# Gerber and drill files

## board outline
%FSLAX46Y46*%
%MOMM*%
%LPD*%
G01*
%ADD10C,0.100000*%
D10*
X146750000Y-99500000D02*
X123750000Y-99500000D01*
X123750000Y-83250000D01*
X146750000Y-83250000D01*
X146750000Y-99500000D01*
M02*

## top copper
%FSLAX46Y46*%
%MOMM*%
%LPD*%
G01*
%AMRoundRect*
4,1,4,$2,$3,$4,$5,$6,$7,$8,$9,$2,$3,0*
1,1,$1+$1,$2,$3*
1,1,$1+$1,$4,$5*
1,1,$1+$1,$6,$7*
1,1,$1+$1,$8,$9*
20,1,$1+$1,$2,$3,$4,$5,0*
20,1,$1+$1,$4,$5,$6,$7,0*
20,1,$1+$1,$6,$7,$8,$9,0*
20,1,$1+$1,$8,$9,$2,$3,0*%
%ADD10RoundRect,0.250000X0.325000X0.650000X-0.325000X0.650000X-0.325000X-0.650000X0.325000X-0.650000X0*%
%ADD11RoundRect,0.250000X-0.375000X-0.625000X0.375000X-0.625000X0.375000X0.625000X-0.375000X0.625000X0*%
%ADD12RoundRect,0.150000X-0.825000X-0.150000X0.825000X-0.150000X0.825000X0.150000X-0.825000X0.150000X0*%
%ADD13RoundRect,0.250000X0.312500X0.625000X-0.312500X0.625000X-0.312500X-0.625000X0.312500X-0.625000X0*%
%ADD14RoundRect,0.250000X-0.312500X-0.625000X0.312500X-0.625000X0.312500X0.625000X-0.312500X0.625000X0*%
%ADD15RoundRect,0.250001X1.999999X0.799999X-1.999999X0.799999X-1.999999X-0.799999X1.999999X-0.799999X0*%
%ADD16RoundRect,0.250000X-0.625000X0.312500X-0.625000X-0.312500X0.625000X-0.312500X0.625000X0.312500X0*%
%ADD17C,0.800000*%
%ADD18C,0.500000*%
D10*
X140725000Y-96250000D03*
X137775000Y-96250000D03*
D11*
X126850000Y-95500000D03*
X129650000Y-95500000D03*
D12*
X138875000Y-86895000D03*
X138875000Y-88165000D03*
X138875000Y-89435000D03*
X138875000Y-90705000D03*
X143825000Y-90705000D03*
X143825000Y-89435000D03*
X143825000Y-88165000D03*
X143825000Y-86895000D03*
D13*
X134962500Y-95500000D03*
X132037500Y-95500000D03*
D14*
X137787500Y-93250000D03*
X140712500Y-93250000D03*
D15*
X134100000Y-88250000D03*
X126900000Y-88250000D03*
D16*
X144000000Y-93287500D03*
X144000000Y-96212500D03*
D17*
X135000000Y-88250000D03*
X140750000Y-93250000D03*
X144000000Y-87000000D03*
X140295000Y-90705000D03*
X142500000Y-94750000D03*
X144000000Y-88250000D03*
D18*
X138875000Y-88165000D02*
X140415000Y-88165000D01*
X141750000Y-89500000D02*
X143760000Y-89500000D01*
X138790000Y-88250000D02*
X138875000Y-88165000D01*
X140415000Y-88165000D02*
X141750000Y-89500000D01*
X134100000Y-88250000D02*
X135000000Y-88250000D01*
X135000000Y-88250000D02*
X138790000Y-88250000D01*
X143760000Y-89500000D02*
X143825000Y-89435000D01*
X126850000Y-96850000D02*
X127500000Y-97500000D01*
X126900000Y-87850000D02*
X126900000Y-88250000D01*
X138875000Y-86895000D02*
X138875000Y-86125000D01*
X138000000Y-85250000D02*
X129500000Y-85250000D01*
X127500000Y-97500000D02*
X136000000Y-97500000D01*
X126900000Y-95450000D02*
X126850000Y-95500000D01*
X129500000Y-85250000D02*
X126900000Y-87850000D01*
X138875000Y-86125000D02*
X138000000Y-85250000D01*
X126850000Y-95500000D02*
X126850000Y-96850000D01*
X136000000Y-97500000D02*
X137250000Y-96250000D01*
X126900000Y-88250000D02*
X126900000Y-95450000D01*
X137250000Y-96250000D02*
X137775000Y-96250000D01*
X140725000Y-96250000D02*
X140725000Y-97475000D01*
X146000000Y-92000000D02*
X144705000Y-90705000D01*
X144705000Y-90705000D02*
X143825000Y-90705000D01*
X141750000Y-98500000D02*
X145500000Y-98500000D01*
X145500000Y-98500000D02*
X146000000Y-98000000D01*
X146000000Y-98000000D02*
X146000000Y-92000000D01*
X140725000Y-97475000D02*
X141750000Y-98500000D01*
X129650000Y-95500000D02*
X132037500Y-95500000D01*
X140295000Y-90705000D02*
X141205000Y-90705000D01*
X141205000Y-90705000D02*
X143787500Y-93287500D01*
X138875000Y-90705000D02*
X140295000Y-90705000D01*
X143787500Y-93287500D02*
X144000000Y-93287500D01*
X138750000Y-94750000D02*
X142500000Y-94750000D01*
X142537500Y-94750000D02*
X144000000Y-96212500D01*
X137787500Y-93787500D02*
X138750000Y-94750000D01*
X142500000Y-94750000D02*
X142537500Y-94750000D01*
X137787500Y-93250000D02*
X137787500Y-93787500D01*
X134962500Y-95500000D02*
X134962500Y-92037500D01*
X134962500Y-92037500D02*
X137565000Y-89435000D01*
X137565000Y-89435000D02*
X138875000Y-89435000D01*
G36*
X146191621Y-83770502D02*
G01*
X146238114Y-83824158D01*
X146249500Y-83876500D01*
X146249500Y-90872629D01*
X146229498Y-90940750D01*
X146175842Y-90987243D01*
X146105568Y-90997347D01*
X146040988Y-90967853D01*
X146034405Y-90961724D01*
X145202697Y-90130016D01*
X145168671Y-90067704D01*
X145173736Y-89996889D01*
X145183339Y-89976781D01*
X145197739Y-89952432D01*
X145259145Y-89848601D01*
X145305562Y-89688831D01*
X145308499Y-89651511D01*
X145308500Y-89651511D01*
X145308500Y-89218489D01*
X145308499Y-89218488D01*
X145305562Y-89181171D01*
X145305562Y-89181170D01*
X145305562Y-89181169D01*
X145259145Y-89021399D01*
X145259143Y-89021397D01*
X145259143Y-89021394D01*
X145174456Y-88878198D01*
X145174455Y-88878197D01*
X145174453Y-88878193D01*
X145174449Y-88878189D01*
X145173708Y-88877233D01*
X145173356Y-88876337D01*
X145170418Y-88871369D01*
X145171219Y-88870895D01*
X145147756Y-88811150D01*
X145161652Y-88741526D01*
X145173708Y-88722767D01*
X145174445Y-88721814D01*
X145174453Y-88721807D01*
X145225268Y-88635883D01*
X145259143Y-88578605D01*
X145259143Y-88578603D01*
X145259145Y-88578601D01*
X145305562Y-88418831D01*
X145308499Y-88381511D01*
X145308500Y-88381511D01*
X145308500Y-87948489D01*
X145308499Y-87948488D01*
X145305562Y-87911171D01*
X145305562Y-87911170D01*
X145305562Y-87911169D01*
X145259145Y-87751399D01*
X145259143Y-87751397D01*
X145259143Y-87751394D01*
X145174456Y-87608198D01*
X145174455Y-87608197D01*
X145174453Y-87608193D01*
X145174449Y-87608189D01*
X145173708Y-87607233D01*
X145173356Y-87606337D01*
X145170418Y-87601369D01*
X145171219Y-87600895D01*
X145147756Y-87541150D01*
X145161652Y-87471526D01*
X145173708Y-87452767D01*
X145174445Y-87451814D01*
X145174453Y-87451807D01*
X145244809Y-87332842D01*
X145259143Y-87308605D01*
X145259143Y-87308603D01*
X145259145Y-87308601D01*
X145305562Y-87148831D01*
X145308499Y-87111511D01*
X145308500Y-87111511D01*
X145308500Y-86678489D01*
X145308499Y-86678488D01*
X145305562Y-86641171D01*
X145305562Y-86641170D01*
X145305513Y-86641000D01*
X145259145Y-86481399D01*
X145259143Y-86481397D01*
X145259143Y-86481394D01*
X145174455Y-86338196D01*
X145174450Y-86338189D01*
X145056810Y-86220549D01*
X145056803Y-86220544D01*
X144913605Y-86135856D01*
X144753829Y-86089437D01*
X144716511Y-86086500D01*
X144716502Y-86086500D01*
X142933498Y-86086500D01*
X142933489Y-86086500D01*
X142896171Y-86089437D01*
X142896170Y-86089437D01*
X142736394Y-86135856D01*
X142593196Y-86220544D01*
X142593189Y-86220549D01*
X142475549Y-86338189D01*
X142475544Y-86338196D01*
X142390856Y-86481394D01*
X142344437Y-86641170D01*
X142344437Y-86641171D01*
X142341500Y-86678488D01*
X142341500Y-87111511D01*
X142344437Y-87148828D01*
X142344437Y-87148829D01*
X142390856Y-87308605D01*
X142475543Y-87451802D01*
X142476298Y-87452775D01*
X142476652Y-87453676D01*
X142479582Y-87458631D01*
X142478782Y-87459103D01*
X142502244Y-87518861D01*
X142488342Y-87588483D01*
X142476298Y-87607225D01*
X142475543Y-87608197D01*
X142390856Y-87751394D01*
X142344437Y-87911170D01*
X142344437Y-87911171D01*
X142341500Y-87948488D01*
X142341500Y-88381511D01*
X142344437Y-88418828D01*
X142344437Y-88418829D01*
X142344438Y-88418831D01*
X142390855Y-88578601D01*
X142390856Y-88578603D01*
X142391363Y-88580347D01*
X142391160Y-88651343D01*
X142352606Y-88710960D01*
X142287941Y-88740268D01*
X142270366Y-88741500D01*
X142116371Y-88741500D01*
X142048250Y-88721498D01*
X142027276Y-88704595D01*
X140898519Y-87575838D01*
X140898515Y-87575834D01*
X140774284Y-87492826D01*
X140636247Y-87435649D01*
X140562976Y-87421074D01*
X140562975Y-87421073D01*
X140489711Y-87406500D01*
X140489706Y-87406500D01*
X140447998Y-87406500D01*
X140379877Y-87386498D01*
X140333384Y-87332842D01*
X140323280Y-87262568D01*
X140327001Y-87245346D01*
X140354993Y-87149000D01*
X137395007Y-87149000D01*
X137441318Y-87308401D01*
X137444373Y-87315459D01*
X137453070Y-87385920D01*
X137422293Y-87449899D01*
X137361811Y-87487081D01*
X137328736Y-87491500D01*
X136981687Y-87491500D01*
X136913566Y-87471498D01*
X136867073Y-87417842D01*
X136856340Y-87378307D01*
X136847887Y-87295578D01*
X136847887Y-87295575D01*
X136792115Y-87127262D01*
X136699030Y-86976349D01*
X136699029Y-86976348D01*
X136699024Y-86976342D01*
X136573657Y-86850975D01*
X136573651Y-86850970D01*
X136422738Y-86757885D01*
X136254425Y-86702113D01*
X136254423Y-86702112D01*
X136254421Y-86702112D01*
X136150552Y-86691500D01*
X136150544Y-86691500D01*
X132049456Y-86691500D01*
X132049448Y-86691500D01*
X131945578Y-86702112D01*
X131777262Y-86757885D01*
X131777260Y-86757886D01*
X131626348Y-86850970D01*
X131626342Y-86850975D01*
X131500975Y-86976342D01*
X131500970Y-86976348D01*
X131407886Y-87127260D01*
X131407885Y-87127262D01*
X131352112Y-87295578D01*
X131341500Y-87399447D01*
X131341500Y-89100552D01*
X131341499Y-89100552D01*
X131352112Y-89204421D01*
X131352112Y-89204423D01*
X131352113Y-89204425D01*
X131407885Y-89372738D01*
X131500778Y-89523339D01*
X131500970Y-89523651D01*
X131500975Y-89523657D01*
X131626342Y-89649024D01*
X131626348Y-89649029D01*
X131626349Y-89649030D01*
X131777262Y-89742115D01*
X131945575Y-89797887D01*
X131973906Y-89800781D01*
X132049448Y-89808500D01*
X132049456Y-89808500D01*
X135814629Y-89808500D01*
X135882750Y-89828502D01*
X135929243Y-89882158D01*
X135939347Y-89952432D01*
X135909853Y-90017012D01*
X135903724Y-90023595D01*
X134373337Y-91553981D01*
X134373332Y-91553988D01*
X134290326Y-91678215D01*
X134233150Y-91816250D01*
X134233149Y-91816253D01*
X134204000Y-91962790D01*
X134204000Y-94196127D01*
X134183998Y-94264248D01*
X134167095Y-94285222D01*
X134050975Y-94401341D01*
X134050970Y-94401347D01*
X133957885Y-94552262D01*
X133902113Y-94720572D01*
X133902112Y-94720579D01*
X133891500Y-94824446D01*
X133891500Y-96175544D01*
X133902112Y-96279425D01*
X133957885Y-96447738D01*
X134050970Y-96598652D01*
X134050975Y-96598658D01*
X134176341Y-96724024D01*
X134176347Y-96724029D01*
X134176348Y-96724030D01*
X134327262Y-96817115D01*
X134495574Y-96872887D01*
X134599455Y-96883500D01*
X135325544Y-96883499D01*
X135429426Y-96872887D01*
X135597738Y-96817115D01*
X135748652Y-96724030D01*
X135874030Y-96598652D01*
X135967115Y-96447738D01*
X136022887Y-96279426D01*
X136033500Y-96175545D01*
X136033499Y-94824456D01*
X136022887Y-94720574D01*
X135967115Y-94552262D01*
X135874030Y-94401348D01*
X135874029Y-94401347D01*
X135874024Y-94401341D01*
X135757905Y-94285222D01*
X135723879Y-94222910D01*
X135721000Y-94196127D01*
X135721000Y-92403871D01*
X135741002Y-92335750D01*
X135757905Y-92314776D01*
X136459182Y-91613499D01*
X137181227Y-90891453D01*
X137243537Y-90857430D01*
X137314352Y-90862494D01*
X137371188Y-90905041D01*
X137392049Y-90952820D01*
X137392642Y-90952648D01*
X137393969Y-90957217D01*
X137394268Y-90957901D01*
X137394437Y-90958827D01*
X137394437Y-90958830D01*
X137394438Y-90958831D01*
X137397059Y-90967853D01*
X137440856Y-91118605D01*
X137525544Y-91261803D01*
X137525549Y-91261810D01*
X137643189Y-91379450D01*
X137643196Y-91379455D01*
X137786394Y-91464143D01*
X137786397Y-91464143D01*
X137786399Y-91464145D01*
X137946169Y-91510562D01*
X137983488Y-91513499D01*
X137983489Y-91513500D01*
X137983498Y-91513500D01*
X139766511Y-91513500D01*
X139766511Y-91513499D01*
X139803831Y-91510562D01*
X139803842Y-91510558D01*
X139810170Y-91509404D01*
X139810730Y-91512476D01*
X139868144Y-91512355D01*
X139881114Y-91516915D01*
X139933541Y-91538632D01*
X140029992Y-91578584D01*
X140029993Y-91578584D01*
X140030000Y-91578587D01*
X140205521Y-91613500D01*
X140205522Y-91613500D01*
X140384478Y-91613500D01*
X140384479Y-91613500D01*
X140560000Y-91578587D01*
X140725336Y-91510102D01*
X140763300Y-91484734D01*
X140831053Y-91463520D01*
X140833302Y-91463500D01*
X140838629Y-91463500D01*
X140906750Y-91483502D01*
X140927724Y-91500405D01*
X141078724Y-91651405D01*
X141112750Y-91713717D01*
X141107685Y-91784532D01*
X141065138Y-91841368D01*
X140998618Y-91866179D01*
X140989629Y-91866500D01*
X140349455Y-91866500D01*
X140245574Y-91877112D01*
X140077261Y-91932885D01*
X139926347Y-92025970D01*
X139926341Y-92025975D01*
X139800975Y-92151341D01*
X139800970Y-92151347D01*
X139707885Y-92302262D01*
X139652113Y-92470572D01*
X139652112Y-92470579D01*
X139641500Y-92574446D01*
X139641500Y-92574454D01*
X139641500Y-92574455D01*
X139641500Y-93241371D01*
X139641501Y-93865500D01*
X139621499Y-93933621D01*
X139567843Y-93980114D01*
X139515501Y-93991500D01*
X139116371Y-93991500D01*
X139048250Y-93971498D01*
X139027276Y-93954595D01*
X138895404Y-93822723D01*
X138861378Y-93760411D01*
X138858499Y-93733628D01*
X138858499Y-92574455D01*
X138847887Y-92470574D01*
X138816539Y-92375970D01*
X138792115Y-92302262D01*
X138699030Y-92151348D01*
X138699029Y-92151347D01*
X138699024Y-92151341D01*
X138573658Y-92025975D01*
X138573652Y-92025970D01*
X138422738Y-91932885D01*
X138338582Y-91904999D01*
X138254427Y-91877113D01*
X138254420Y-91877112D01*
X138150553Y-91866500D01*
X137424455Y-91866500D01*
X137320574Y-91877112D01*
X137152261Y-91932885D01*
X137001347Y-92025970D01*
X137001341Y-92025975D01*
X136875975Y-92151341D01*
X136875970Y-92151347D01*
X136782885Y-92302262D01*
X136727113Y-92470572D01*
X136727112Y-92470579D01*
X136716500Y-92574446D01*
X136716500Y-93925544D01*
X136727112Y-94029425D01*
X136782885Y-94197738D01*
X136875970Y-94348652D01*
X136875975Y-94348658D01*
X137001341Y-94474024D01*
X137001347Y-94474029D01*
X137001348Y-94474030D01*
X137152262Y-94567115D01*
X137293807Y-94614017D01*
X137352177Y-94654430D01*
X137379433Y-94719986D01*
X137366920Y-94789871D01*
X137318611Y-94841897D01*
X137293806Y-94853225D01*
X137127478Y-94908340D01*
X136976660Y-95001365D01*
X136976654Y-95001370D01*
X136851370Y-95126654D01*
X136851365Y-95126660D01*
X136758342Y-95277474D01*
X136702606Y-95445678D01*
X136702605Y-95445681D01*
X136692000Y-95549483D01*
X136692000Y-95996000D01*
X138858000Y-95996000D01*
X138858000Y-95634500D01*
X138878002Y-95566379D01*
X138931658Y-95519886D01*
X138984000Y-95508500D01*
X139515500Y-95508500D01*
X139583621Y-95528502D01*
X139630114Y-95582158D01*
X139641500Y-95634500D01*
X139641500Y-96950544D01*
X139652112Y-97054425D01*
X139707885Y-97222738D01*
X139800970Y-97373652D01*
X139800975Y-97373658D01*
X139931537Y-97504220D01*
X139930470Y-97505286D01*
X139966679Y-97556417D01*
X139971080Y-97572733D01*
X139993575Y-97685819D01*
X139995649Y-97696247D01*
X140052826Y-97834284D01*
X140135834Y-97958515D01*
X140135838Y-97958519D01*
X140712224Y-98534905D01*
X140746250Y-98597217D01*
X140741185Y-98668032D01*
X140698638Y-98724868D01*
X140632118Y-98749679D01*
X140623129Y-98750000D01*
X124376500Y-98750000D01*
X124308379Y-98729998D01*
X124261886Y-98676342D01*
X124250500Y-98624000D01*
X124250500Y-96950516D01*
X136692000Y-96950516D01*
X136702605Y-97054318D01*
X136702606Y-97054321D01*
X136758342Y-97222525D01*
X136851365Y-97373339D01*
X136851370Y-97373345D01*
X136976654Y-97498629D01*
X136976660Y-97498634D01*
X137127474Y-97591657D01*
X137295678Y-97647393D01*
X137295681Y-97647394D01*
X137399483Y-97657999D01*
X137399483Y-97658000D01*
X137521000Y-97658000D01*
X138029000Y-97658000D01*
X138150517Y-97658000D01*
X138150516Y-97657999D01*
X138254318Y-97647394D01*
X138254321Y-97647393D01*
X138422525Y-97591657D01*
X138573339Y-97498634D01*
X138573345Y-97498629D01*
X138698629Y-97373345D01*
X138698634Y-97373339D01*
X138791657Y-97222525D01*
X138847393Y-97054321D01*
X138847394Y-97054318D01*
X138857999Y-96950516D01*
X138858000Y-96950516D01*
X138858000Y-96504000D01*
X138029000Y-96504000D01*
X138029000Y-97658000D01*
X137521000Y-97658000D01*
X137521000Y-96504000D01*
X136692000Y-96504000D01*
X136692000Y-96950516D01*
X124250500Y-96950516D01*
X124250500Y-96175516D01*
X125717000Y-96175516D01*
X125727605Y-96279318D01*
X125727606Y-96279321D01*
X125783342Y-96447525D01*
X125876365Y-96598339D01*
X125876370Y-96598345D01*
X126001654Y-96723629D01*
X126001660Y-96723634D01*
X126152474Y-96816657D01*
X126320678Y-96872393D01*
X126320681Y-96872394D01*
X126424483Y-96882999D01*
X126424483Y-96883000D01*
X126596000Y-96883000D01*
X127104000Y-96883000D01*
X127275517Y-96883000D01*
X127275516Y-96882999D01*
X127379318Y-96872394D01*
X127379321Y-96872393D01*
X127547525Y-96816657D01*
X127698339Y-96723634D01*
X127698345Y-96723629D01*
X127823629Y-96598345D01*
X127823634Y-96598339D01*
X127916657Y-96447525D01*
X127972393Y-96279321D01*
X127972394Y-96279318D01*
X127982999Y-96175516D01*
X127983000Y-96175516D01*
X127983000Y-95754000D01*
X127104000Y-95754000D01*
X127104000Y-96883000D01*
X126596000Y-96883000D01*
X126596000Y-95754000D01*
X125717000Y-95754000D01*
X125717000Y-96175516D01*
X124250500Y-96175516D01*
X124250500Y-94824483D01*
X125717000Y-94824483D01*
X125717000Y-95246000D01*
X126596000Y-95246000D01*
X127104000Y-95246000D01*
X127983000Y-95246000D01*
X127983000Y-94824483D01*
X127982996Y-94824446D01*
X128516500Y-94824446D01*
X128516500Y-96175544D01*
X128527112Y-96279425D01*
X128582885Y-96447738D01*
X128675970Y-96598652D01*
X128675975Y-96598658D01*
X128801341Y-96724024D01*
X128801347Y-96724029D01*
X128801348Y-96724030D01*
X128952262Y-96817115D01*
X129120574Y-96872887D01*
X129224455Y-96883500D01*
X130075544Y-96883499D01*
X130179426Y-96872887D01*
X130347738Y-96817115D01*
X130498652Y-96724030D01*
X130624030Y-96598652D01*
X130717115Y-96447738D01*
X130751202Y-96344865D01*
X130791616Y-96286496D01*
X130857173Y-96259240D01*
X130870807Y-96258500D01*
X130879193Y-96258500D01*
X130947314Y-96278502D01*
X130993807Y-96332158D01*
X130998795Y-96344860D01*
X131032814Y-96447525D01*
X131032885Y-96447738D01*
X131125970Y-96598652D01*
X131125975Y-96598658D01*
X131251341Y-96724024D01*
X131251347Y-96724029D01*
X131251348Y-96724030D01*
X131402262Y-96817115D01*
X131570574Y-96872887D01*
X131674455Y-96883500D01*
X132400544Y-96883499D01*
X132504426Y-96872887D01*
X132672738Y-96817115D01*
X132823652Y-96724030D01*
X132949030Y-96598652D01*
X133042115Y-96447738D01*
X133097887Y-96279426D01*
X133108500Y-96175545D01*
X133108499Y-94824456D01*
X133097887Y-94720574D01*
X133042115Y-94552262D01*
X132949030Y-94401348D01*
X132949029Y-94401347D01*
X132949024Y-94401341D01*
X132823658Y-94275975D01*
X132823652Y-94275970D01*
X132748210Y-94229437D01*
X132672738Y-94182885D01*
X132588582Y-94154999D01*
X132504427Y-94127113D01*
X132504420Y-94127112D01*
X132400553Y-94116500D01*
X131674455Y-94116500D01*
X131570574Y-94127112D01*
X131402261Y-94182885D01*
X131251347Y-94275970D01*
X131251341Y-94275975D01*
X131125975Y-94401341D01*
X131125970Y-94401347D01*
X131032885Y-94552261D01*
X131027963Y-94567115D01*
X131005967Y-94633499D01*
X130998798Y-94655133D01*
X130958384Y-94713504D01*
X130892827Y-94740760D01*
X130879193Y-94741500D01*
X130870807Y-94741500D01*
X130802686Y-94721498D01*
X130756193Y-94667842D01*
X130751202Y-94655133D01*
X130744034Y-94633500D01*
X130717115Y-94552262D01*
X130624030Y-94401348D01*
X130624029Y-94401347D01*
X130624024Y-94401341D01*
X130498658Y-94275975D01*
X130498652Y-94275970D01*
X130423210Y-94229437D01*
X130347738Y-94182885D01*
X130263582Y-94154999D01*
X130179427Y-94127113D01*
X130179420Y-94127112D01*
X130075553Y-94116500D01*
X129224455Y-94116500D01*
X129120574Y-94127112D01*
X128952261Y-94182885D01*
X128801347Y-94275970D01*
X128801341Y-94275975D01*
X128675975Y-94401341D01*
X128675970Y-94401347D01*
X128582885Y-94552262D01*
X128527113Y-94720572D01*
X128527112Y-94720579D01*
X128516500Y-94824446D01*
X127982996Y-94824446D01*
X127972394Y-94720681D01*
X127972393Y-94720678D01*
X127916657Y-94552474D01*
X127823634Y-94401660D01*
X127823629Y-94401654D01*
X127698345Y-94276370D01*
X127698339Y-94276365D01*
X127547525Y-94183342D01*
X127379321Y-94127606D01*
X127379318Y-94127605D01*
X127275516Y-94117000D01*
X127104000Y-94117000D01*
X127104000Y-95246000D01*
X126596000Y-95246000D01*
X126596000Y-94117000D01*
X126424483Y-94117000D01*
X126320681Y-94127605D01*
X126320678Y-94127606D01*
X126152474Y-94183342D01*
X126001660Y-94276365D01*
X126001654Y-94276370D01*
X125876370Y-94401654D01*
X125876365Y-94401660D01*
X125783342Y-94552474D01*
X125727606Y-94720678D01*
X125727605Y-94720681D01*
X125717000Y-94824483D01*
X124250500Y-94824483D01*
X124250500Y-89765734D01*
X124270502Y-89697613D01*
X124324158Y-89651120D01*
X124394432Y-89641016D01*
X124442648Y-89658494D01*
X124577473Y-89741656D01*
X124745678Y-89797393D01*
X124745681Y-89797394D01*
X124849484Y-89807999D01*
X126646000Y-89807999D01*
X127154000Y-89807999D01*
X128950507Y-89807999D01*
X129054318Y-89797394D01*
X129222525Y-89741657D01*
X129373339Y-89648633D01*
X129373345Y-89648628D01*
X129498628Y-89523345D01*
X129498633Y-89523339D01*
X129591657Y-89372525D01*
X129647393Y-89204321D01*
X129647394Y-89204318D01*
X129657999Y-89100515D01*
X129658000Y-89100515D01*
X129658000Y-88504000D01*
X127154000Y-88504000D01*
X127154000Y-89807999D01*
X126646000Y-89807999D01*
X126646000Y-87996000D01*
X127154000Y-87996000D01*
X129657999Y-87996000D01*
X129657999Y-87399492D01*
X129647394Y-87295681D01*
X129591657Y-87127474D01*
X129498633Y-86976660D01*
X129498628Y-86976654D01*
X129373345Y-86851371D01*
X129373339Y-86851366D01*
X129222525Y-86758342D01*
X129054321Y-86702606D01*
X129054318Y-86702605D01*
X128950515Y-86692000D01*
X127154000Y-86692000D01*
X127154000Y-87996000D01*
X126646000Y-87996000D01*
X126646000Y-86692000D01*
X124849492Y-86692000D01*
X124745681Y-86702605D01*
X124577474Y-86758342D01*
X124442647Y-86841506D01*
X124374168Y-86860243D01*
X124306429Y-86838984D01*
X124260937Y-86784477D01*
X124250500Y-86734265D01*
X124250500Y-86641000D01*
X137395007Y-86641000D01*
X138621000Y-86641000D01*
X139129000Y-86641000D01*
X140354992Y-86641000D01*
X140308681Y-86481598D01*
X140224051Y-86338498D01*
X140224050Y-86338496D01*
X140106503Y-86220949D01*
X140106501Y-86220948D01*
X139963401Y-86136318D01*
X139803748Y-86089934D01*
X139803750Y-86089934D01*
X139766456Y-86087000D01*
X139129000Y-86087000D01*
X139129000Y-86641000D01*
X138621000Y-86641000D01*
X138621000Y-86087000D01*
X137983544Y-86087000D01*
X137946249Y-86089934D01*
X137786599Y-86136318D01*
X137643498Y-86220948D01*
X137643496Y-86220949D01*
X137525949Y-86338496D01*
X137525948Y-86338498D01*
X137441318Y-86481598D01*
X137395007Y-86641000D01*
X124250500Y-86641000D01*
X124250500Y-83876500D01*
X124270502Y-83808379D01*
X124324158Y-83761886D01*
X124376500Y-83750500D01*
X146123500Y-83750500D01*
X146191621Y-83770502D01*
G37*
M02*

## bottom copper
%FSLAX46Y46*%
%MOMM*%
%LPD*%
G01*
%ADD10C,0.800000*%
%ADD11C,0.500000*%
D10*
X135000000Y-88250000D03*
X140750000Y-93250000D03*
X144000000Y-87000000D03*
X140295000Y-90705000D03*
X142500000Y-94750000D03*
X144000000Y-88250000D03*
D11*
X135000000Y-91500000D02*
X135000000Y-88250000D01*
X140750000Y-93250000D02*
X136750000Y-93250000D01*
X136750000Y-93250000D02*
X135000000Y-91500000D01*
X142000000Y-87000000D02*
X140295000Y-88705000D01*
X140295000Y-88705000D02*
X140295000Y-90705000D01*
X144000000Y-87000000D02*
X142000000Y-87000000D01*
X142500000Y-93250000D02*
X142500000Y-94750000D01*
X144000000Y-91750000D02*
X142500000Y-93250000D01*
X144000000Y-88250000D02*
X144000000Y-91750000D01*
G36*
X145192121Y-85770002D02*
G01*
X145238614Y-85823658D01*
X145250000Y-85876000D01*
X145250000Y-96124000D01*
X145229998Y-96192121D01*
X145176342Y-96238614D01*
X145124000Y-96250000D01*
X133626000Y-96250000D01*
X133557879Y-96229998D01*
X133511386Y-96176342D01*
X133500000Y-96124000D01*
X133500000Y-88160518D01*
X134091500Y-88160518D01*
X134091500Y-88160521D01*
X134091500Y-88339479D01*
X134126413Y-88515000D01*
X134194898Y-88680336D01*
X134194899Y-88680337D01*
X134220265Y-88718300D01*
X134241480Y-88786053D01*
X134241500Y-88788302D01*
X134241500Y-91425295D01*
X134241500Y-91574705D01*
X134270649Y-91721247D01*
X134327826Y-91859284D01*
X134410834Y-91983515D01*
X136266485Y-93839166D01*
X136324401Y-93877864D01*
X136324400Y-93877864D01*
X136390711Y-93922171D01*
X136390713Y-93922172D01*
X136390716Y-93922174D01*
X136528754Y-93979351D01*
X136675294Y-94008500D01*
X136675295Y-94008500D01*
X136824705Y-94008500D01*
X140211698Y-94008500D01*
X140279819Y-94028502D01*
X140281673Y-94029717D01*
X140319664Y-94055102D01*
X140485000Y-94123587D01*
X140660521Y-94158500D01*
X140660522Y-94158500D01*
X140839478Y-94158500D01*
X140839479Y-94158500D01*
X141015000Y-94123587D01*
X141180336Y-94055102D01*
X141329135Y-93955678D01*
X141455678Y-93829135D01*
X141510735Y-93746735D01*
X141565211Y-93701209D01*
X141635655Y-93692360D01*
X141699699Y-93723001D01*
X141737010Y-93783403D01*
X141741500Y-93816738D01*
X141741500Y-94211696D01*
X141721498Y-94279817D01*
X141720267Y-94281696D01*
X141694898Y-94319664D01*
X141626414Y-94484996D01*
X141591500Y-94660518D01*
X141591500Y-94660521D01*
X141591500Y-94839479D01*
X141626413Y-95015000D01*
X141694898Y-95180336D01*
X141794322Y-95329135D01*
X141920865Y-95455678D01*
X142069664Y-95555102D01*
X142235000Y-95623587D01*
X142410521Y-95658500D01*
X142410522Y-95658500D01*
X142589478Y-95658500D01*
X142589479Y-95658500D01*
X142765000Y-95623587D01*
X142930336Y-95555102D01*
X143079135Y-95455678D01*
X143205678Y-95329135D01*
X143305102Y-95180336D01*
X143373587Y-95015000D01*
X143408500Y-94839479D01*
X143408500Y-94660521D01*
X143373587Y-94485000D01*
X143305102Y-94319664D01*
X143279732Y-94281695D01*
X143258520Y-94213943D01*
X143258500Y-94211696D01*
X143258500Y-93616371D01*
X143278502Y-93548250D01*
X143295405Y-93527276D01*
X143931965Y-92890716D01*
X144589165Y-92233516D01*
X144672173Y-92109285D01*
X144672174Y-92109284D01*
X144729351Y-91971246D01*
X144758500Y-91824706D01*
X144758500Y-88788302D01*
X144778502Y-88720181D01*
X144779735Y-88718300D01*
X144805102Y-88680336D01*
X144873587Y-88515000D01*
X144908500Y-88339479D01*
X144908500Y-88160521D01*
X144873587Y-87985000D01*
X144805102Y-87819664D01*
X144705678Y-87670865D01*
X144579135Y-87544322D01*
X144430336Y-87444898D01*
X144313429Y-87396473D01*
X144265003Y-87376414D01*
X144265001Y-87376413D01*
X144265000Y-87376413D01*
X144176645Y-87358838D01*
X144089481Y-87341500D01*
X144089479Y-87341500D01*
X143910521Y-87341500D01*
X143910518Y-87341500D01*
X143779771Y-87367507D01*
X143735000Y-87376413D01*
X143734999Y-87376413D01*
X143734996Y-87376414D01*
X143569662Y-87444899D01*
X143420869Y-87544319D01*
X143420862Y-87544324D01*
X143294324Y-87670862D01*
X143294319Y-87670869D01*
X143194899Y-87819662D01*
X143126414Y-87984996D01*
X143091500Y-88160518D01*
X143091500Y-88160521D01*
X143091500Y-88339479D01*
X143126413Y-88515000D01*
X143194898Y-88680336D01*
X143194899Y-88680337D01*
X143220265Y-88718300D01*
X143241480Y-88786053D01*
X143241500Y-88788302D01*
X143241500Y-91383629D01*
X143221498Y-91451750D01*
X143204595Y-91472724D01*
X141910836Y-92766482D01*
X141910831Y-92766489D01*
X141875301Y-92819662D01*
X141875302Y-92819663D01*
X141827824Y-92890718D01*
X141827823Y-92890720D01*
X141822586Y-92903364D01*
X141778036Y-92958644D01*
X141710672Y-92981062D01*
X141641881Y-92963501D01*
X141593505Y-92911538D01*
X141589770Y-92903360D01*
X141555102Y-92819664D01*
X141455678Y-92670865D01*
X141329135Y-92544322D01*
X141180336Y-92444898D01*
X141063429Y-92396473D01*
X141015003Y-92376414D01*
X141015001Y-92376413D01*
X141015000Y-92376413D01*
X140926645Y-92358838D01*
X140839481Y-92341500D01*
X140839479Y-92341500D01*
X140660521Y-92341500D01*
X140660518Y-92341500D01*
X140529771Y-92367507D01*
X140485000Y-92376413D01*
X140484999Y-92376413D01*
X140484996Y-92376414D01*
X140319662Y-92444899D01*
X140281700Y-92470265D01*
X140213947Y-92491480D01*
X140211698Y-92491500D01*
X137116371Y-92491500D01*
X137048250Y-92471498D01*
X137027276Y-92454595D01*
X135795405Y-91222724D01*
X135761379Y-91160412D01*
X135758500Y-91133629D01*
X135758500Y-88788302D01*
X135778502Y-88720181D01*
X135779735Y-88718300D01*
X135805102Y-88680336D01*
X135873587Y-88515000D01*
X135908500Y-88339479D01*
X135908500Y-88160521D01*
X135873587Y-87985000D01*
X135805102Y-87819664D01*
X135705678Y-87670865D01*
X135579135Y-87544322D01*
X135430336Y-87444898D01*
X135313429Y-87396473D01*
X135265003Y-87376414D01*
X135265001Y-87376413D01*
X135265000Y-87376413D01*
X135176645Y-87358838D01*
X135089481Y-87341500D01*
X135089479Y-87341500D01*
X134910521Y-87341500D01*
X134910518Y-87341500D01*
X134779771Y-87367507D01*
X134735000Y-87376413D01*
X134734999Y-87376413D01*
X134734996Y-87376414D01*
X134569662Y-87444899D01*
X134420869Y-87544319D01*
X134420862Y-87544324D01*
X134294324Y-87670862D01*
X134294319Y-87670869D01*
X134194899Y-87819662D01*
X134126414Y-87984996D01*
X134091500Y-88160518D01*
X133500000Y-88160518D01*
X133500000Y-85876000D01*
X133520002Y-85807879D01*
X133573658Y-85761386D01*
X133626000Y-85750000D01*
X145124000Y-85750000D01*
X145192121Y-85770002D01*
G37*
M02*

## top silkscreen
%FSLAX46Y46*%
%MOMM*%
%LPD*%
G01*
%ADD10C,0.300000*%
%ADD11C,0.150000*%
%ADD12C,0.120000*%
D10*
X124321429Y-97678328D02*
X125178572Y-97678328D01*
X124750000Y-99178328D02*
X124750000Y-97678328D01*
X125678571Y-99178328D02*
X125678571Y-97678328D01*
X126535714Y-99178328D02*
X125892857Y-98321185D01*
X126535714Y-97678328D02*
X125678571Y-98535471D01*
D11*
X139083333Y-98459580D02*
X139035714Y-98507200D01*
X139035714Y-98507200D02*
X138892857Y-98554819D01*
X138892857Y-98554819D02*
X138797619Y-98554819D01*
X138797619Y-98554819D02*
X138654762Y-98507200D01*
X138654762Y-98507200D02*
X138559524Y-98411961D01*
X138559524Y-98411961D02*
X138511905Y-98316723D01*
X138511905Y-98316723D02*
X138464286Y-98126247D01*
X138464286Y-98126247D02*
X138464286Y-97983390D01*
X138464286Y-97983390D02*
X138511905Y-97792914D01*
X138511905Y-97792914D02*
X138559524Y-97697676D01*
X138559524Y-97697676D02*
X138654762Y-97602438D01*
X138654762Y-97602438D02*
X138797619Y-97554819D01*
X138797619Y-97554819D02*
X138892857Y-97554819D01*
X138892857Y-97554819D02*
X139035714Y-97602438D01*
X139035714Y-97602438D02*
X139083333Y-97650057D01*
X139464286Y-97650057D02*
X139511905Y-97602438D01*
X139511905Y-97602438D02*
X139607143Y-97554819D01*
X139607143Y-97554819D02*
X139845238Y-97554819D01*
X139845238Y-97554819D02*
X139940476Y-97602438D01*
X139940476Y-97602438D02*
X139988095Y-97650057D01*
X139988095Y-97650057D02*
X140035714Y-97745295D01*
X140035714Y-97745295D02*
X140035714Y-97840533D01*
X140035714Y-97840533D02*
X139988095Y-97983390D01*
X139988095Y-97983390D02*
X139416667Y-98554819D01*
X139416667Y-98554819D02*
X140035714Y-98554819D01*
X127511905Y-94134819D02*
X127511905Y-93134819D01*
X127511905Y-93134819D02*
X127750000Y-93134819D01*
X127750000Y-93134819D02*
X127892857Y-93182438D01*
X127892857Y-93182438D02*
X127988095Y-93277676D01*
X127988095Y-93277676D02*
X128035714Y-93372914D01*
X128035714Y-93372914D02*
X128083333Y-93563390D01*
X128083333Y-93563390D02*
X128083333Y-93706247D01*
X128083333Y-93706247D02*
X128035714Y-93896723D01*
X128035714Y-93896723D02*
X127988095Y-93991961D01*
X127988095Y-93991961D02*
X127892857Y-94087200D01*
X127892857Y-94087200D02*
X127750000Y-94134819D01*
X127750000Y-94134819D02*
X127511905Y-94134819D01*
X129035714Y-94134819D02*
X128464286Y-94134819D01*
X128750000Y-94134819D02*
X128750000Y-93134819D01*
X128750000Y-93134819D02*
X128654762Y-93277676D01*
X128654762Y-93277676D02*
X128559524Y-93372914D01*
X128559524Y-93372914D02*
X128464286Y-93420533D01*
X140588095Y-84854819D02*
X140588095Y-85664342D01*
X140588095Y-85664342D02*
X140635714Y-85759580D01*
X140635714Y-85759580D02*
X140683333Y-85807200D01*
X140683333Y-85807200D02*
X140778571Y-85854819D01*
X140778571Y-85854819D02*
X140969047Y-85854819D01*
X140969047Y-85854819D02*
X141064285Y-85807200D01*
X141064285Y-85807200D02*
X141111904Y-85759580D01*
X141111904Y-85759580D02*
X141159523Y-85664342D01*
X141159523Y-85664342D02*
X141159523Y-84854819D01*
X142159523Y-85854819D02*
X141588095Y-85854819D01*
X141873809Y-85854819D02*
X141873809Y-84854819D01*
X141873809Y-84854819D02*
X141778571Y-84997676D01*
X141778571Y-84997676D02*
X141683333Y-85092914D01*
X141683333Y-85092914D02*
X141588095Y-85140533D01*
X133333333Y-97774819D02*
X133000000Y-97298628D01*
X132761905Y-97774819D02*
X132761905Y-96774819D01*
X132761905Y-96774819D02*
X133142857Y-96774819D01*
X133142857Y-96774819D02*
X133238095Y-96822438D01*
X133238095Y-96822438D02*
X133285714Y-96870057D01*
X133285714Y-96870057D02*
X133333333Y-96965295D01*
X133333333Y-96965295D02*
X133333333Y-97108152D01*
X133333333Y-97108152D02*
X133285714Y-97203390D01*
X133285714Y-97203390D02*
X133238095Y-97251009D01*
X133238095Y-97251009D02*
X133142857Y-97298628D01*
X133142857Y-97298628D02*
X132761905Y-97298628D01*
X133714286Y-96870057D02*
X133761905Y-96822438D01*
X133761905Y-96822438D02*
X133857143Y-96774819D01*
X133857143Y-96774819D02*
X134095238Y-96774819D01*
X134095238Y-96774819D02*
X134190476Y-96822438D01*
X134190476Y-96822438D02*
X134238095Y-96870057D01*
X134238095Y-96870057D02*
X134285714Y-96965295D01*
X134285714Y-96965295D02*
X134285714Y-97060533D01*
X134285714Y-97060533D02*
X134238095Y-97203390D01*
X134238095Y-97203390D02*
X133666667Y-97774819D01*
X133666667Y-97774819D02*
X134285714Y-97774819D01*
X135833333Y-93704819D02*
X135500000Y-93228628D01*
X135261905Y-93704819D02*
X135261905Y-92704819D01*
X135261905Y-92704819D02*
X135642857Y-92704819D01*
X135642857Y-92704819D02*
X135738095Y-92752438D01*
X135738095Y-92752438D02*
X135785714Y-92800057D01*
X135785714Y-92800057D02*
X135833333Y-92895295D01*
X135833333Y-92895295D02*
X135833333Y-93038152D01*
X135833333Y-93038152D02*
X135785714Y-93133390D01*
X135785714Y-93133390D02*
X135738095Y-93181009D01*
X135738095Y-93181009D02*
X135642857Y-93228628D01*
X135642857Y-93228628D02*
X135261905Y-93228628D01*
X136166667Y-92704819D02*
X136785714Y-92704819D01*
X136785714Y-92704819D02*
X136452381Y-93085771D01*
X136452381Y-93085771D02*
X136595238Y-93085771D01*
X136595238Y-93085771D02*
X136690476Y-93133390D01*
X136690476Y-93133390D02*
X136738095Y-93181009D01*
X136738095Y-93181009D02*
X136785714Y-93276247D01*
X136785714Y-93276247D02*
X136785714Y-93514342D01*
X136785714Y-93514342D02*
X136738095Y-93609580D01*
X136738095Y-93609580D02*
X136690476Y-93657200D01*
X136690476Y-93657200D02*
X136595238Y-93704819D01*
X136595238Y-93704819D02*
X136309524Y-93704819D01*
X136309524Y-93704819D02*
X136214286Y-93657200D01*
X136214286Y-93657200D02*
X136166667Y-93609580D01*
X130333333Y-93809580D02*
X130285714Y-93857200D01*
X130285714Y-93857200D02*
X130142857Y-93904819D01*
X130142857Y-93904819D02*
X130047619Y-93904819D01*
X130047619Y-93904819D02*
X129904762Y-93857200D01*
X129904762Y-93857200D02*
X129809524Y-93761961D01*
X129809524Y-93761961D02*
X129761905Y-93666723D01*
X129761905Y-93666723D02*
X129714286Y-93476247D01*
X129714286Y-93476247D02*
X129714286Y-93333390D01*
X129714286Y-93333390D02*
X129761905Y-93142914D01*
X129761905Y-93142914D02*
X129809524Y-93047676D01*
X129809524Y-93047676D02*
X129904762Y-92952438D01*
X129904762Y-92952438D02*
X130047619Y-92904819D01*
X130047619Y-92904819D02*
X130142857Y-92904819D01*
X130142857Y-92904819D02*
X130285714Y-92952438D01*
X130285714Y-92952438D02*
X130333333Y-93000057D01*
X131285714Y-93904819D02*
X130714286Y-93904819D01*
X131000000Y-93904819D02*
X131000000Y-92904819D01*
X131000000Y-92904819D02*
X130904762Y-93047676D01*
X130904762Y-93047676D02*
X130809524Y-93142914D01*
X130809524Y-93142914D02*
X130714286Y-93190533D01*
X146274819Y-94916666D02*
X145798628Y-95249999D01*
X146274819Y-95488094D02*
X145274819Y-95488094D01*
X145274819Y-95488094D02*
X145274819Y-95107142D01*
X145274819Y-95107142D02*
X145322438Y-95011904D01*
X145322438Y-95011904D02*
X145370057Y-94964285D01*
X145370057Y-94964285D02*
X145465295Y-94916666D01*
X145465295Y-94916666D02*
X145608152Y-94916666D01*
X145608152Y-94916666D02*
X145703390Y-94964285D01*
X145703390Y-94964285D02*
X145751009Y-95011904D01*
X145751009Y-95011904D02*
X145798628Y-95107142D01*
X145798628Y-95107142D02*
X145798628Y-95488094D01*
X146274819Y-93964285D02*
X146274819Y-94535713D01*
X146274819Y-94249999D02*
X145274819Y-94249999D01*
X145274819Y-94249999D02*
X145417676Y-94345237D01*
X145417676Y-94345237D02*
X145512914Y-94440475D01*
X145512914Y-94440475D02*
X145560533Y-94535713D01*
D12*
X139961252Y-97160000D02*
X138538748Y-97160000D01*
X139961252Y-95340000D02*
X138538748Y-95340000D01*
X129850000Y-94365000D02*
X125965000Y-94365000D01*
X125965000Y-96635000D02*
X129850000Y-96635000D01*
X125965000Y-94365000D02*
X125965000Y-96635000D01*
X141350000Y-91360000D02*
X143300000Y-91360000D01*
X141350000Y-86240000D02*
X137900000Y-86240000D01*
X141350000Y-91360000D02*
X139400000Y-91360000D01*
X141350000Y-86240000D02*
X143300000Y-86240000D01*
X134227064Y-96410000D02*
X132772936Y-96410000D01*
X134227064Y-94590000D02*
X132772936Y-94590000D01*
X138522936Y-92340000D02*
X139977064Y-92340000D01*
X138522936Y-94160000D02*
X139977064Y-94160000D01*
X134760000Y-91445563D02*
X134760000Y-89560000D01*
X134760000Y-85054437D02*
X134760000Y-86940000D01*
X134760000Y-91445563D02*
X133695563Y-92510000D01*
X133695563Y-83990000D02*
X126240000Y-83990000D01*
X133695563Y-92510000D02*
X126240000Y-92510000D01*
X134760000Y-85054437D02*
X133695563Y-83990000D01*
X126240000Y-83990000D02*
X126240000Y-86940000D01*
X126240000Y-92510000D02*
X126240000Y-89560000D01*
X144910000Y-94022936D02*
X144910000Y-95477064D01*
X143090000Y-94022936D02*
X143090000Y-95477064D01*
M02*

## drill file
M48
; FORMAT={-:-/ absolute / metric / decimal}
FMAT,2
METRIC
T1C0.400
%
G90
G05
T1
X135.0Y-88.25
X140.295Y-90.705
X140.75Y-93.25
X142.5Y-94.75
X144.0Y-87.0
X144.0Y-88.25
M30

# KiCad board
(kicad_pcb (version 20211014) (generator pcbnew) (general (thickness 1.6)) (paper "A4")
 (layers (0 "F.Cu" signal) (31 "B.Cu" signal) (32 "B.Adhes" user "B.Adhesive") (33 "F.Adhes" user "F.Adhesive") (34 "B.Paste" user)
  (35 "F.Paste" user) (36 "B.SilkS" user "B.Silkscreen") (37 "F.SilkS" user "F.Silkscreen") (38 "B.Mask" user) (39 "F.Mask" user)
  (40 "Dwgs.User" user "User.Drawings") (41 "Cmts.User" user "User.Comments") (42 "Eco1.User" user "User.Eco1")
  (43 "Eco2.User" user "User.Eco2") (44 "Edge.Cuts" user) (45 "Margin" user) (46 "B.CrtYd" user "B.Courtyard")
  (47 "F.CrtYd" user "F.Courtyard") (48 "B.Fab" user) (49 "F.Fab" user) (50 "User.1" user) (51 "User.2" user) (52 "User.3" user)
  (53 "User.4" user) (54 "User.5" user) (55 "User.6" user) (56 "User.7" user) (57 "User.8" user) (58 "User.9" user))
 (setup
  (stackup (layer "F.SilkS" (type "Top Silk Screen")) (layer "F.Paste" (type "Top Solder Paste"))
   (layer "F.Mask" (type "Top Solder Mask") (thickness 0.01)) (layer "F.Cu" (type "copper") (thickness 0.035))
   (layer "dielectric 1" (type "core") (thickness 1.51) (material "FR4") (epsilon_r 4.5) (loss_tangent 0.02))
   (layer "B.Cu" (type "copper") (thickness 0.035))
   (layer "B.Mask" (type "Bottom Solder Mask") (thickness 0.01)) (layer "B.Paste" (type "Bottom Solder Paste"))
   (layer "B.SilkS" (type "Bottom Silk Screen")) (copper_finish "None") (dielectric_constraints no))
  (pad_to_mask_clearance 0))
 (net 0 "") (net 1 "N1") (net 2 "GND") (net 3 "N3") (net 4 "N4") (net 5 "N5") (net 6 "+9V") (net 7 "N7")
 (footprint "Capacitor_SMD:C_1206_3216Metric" (layer "F.Cu") (at 139.25 96.25 180)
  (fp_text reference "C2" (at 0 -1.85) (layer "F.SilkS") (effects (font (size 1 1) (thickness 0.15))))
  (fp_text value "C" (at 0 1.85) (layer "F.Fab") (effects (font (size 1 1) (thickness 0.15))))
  (fp_line (start -0.711252 -0.91) (end 0.711252 -0.91) (layer "F.SilkS") (width 0.12))
  (fp_line (start -0.711252 0.91) (end 0.711252 0.91) (layer "F.SilkS") (width 0.12))
  (pad "1" smd roundrect (at -1.475 0 180) (size 1.15 1.8) (layers "F.Cu" "F.Paste" "F.Mask") (roundrect_rratio 0.2173913043) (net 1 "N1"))
  (pad "2" smd roundrect (at 1.475 0 180) (size 1.15 1.8) (layers "F.Cu" "F.Paste" "F.Mask") (roundrect_rratio 0.2173913043) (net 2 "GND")))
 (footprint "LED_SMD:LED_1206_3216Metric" (layer "F.Cu") (at 128.25 95.5)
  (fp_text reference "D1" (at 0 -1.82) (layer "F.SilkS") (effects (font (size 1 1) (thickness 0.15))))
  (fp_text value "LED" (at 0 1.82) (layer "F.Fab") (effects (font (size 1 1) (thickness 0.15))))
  (fp_line (start 1.6 -1.135) (end -2.285 -1.135) (layer "F.SilkS") (width 0.12))
  (fp_line (start -2.285 1.135) (end 1.6 1.135) (layer "F.SilkS") (width 0.12))
  (fp_line (start -2.285 -1.135) (end -2.285 1.135) (layer "F.SilkS") (width 0.12))
  (pad "1" smd roundrect (at -1.4 0) (size 1.25 1.75) (layers "F.Cu" "F.Paste" "F.Mask") (roundrect_rratio 0.2) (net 2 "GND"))
  (pad "2" smd roundrect (at 1.4 0) (size 1.25 1.75) (layers "F.Cu" "F.Paste" "F.Mask") (roundrect_rratio 0.2) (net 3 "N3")))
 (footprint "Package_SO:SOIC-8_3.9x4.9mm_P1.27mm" (layer "F.Cu") (at 141.35 88.8)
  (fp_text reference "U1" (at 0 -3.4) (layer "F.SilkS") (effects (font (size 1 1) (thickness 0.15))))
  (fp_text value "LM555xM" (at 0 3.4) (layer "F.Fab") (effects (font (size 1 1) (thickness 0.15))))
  (fp_line (start 0 2.56) (end 1.95 2.56) (layer "F.SilkS") (width 0.12))
  (fp_line (start 0 -2.56) (end -3.45 -2.56) (layer "F.SilkS") (width 0.12))
  (fp_line (start 0 2.56) (end -1.95 2.56) (layer "F.SilkS") (width 0.12))
  (fp_line (start 0 -2.56) (end 1.95 -2.56) (layer "F.SilkS") (width 0.12))
  (pad "1" smd roundrect (at -2.475 -1.905) (size 1.95 0.6) (layers "F.Cu" "F.Paste" "F.Mask") (roundrect_rratio 0.25) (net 2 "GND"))
  (pad "2" smd roundrect (at -2.475 -0.635) (size 1.95 0.6) (layers "F.Cu" "F.Paste" "F.Mask") (roundrect_rratio 0.25) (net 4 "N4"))
  (pad "3" smd roundrect (at -2.475 0.635) (size 1.95 0.6) (layers "F.Cu" "F.Paste" "F.Mask") (roundrect_rratio 0.25) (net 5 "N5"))
  (pad "4" smd roundrect (at -2.475 1.905) (size 1.95 0.6) (layers "F.Cu" "F.Paste" "F.Mask") (roundrect_rratio 0.25) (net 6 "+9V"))
  (pad "5" smd roundrect (at 2.475 1.905) (size 1.95 0.6) (layers "F.Cu" "F.Paste" "F.Mask") (roundrect_rratio 0.25) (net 1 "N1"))
  (pad "6" smd roundrect (at 2.475 0.635) (size 1.95 0.6) (layers "F.Cu" "F.Paste" "F.Mask") (roundrect_rratio 0.25) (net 4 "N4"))
  (pad "7" smd roundrect (at 2.475 -0.635) (size 1.95 0.6) (layers "F.Cu" "F.Paste" "F.Mask") (roundrect_rratio 0.25) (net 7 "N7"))
  (pad "8" smd roundrect (at 2.475 -1.905) (size 1.95 0.6) (layers "F.Cu" "F.Paste" "F.Mask") (roundrect_rratio 0.25) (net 6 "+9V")))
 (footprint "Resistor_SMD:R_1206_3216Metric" (layer "F.Cu") (at 133.5 95.5 180)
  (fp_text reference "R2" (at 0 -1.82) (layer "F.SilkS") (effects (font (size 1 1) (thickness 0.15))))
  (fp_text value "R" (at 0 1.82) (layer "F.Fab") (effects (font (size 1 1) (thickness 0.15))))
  (fp_line (start -0.727064 -0.91) (end 0.727064 -0.91) (layer "F.SilkS") (width 0.12))
  (fp_line (start -0.727064 0.91) (end 0.727064 0.91) (layer "F.SilkS") (width 0.12))
  (pad "1" smd roundrect (at -1.4625 0 180) (size 1.125 1.75) (layers "F.Cu" "F.Paste" "F.Mask") (roundrect_rratio 0.2222222222)
   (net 5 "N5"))
  (pad "2" smd roundrect (at 1.4625 0 180) (size 1.125 1.75) (layers "F.Cu" "F.Paste" "F.Mask") (roundrect_rratio 0.2222222222) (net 3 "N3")))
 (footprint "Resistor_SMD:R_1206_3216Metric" (layer "F.Cu") (at 139.25 93.25)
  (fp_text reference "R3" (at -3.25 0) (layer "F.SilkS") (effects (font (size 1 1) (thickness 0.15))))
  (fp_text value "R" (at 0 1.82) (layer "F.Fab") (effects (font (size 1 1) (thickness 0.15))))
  (fp_line (start -0.727064 -0.91) (end 0.727064 -0.91) (layer "F.SilkS") (width 0.12))
  (fp_line (start -0.727064 0.91) (end 0.727064 0.91) (layer "F.SilkS") (width 0.12))
  (pad "1" smd roundrect (at -1.4625 0) (size 1.125 1.75) (layers "F.Cu" "F.Paste" "F.Mask") (roundrect_rratio 0.2222222222) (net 7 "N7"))
  (pad "2" smd roundrect (at 1.4625 0) (size 1.125 1.75) (layers "F.Cu" "F.Paste" "F.Mask") (roundrect_rratio 0.2222222222) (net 4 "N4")))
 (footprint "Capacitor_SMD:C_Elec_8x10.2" (layer "F.Cu") (at 130.5 88.25 180)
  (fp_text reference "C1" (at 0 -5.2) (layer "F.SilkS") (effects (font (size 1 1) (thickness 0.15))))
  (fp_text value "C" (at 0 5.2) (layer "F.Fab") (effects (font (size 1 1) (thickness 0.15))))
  (fp_line (start -4.26 -3.195563) (end -4.26 -1.31) (layer "F.SilkS") (width 0.12))
  (fp_line (start -4.26 3.195563) (end -4.26 1.31) (layer "F.SilkS") (width 0.12))
  (fp_line (start -4.26 -3.195563) (end -3.195563 -4.26) (layer "F.SilkS") (width 0.12))
  (fp_line (start -3.195563 4.26) (end 4.26 4.26) (layer "F.SilkS") (width 0.12))
  (fp_line (start -3.195563 -4.26) (end 4.26 -4.26) (layer "F.SilkS") (width 0.12))
  (fp_line (start -4.26 3.195563) (end -3.195563 4.26) (layer "F.SilkS") (width 0.12))
  (fp_line (start 4.26 4.26) (end 4.26 1.31) (layer "F.SilkS") (width 0.12))
  (fp_line (start 4.26 -4.26) (end 4.26 -1.31) (layer "F.SilkS") (width 0.12))
  (pad "1" smd roundrect (at -3.6 0 180) (size 4.5 2.1) (layers "F.Cu" "F.Paste" "F.Mask") (roundrect_rratio 0.1190480952) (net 4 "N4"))
  (pad "2" smd roundrect (at 3.6 0 180) (size 4.5 2.1) (layers "F.Cu" "F.Paste" "F.Mask") (roundrect_rratio 0.1190480952) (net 2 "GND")))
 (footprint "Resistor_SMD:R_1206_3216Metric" (layer "F.Cu") (at 144 94.75 -90)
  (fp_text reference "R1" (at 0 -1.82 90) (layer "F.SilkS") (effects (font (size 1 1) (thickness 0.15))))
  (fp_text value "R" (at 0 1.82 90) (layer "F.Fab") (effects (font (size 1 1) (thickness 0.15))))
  (fp_line (start -0.727064 -0.91) (end 0.727064 -0.91) (layer "F.SilkS") (width 0.12))
  (fp_line (start -0.727064 0.91) (end 0.727064 0.91) (layer "F.SilkS") (width 0.12))
  (pad "1" smd roundrect (at -1.4625 0 270) (size 1.125 1.75) (layers "F.Cu" "F.Paste" "F.Mask") (roundrect_rratio 0.2222222222)
   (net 6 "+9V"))
  (pad "2" smd roundrect (at 1.4625 0 270) (size 1.125 1.75) (layers "F.Cu" "F.Paste" "F.Mask") (roundrect_rratio 0.2222222222) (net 7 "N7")))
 (gr_poly (pts (xy 146.75 99.5) (xy 123.75 99.5) (xy 123.75 83.25) (xy 146.75 83.25)) (layer "Edge.Cuts") (width 0.1) (fill none))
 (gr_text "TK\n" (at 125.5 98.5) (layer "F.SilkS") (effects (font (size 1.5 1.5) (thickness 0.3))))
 (segment (start 138.875 88.165) (end 140.415 88.165) (width 0.5) (layer "F.Cu") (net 4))
 (segment (start 141.75 89.5) (end 143.76 89.5) (width 0.5) (layer "F.Cu") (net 4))
 (segment (start 138.79 88.25) (end 138.875 88.165) (width 0.5) (layer "F.Cu") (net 4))
 (segment (start 140.415 88.165) (end 141.75 89.5) (width 0.5) (layer "F.Cu") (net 4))
 (segment (start 134.1 88.25) (end 135 88.25) (width 0.5) (layer "F.Cu") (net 4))
 (segment (start 135 88.25) (end 138.79 88.25) (width 0.5) (layer "F.Cu") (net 4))
 (segment (start 143.76 89.5) (end 143.825 89.435) (width 0.5) (layer "F.Cu") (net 4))
 (via (at 135 88.25) (size 0.8) (drill 0.4) (layers "F.Cu" "B.Cu") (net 4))
 (via (at 140.75 93.25) (size 0.8) (drill 0.4) (layers "F.Cu" "B.Cu") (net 4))
 (segment (start 135 91.5) (end 135 88.25) (width 0.5) (layer "B.Cu") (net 4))
 (segment (start 140.75 93.25) (end 136.75 93.25) (width 0.5) (layer "B.Cu") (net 4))
 (segment (start 136.75 93.25) (end 135 91.5) (width 0.5) (layer "B.Cu") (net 4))
 (segment (start 126.85 96.85) (end 127.5 97.5) (width 0.5) (layer "F.Cu") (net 2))
 (segment (start 126.9 87.85) (end 126.9 88.25) (width 0.5) (layer "F.Cu") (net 2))
 (segment (start 138.875 86.895) (end 138.875 86.125) (width 0.5) (layer "F.Cu") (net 2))
 (segment (start 138 85.25) (end 129.5 85.25) (width 0.5) (layer "F.Cu") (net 2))
 (segment (start 127.5 97.5) (end 136 97.5) (width 0.5) (layer "F.Cu") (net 2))
 (segment (start 126.9 95.45) (end 126.85 95.5) (width 0.5) (layer "F.Cu") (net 2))
 (segment (start 129.5 85.25) (end 126.9 87.85) (width 0.5) (layer "F.Cu") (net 2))
 (segment (start 138.875 86.125) (end 138 85.25) (width 0.5) (layer "F.Cu") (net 2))
 (segment (start 126.85 95.5) (end 126.85 96.85) (width 0.5) (layer "F.Cu") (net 2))
 (segment (start 136 97.5) (end 137.25 96.25) (width 0.5) (layer "F.Cu") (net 2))
 (segment (start 126.9 88.25) (end 126.9 95.45) (width 0.5) (layer "F.Cu") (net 2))
 (segment (start 137.25 96.25) (end 137.775 96.25) (width 0.5) (layer "F.Cu") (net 2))
 (segment (start 140.725 96.25) (end 140.725 97.475) (width 0.5) (layer "F.Cu") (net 1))
 (segment (start 146 92) (end 144.705 90.705) (width 0.5) (layer "F.Cu") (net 1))
 (segment (start 144.705 90.705) (end 143.825 90.705) (width 0.5) (layer "F.Cu") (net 1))
 (segment (start 141.75 98.5) (end 145.5 98.5) (width 0.5) (layer "F.Cu") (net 1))
 (segment (start 145.5 98.5) (end 146 98) (width 0.5) (layer "F.Cu") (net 1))
 (segment (start 146 98) (end 146 92) (width 0.5) (layer "F.Cu") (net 1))
 (segment (start 140.725 97.475) (end 141.75 98.5) (width 0.5) (layer "F.Cu") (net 1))
 (segment (start 129.65 95.5) (end 132.0375 95.5) (width 0.5) (layer "F.Cu") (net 3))
 (segment (start 140.295 90.705) (end 141.205 90.705) (width 0.5) (layer "F.Cu") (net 6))
 (segment (start 141.205 90.705) (end 143.7875 93.2875) (width 0.5) (layer "F.Cu") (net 6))
 (segment (start 138.875 90.705) (end 140.295 90.705) (width 0.5) (layer "F.Cu") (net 6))
 (segment (start 143.7875 93.2875) (end 144 93.2875) (width 0.5) (layer "F.Cu") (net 6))
 (via (at 144 87) (size 0.8) (drill 0.4) (layers "F.Cu" "B.Cu") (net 6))
 (via (at 140.295 90.705) (size 0.8) (drill 0.4) (layers "F.Cu" "B.Cu") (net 6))
 (segment (start 142 87) (end 140.295 88.705) (width 0.5) (layer "B.Cu") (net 6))
 (segment (start 140.295 88.705) (end 140.295 90.705) (width 0.5) (layer "B.Cu") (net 6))
 (segment (start 144 87) (end 142 87) (width 0.5) (layer "B.Cu") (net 6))
 (segment (start 138.75 94.75) (end 142.5 94.75) (width 0.5) (layer "F.Cu") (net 7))
 (segment (start 142.5375 94.75) (end 144 96.2125) (width 0.5) (layer "F.Cu") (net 7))
 (segment (start 137.7875 93.7875) (end 138.75 94.75) (width 0.5) (layer "F.Cu") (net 7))
 (segment (start 142.5 94.75) (end 142.5375 94.75) (width 0.5) (layer "F.Cu") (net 7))
 (segment (start 137.7875 93.25) (end 137.7875 93.7875) (width 0.5) (layer "F.Cu") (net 7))
 (via (at 142.5 94.75) (size 0.8) (drill 0.4) (layers "F.Cu" "B.Cu") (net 7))
 (via (at 144 88.25) (size 0.8) (drill 0.4) (layers "F.Cu" "B.Cu") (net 7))
 (segment (start 142.5 93.25) (end 142.5 94.75) (width 0.5) (layer "B.Cu") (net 7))
 (segment (start 144 91.75) (end 142.5 93.25) (width 0.5) (layer "B.Cu") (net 7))
 (segment (start 144 88.25) (end 144 91.75) (width 0.5) (layer "B.Cu") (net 7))
 (segment (start 134.9625 95.5) (end 134.9625 92.0375) (width 0.5) (layer "F.Cu") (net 5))
 (segment (start 134.9625 92.0375) (end 137.565 89.435) (width 0.5) (layer "F.Cu") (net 5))
 (segment (start 137.565 89.435) (end 138.875 89.435) (width 0.5) (layer "F.Cu") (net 5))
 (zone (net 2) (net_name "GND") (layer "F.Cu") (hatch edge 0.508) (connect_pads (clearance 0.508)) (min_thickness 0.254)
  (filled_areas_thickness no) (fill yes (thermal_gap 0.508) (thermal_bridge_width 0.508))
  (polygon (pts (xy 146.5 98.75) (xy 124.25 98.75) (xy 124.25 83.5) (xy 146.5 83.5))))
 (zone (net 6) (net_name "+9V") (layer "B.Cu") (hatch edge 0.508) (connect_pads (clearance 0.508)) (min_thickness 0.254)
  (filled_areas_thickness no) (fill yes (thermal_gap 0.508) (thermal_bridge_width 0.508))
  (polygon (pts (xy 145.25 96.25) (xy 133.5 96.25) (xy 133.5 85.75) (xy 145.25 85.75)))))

